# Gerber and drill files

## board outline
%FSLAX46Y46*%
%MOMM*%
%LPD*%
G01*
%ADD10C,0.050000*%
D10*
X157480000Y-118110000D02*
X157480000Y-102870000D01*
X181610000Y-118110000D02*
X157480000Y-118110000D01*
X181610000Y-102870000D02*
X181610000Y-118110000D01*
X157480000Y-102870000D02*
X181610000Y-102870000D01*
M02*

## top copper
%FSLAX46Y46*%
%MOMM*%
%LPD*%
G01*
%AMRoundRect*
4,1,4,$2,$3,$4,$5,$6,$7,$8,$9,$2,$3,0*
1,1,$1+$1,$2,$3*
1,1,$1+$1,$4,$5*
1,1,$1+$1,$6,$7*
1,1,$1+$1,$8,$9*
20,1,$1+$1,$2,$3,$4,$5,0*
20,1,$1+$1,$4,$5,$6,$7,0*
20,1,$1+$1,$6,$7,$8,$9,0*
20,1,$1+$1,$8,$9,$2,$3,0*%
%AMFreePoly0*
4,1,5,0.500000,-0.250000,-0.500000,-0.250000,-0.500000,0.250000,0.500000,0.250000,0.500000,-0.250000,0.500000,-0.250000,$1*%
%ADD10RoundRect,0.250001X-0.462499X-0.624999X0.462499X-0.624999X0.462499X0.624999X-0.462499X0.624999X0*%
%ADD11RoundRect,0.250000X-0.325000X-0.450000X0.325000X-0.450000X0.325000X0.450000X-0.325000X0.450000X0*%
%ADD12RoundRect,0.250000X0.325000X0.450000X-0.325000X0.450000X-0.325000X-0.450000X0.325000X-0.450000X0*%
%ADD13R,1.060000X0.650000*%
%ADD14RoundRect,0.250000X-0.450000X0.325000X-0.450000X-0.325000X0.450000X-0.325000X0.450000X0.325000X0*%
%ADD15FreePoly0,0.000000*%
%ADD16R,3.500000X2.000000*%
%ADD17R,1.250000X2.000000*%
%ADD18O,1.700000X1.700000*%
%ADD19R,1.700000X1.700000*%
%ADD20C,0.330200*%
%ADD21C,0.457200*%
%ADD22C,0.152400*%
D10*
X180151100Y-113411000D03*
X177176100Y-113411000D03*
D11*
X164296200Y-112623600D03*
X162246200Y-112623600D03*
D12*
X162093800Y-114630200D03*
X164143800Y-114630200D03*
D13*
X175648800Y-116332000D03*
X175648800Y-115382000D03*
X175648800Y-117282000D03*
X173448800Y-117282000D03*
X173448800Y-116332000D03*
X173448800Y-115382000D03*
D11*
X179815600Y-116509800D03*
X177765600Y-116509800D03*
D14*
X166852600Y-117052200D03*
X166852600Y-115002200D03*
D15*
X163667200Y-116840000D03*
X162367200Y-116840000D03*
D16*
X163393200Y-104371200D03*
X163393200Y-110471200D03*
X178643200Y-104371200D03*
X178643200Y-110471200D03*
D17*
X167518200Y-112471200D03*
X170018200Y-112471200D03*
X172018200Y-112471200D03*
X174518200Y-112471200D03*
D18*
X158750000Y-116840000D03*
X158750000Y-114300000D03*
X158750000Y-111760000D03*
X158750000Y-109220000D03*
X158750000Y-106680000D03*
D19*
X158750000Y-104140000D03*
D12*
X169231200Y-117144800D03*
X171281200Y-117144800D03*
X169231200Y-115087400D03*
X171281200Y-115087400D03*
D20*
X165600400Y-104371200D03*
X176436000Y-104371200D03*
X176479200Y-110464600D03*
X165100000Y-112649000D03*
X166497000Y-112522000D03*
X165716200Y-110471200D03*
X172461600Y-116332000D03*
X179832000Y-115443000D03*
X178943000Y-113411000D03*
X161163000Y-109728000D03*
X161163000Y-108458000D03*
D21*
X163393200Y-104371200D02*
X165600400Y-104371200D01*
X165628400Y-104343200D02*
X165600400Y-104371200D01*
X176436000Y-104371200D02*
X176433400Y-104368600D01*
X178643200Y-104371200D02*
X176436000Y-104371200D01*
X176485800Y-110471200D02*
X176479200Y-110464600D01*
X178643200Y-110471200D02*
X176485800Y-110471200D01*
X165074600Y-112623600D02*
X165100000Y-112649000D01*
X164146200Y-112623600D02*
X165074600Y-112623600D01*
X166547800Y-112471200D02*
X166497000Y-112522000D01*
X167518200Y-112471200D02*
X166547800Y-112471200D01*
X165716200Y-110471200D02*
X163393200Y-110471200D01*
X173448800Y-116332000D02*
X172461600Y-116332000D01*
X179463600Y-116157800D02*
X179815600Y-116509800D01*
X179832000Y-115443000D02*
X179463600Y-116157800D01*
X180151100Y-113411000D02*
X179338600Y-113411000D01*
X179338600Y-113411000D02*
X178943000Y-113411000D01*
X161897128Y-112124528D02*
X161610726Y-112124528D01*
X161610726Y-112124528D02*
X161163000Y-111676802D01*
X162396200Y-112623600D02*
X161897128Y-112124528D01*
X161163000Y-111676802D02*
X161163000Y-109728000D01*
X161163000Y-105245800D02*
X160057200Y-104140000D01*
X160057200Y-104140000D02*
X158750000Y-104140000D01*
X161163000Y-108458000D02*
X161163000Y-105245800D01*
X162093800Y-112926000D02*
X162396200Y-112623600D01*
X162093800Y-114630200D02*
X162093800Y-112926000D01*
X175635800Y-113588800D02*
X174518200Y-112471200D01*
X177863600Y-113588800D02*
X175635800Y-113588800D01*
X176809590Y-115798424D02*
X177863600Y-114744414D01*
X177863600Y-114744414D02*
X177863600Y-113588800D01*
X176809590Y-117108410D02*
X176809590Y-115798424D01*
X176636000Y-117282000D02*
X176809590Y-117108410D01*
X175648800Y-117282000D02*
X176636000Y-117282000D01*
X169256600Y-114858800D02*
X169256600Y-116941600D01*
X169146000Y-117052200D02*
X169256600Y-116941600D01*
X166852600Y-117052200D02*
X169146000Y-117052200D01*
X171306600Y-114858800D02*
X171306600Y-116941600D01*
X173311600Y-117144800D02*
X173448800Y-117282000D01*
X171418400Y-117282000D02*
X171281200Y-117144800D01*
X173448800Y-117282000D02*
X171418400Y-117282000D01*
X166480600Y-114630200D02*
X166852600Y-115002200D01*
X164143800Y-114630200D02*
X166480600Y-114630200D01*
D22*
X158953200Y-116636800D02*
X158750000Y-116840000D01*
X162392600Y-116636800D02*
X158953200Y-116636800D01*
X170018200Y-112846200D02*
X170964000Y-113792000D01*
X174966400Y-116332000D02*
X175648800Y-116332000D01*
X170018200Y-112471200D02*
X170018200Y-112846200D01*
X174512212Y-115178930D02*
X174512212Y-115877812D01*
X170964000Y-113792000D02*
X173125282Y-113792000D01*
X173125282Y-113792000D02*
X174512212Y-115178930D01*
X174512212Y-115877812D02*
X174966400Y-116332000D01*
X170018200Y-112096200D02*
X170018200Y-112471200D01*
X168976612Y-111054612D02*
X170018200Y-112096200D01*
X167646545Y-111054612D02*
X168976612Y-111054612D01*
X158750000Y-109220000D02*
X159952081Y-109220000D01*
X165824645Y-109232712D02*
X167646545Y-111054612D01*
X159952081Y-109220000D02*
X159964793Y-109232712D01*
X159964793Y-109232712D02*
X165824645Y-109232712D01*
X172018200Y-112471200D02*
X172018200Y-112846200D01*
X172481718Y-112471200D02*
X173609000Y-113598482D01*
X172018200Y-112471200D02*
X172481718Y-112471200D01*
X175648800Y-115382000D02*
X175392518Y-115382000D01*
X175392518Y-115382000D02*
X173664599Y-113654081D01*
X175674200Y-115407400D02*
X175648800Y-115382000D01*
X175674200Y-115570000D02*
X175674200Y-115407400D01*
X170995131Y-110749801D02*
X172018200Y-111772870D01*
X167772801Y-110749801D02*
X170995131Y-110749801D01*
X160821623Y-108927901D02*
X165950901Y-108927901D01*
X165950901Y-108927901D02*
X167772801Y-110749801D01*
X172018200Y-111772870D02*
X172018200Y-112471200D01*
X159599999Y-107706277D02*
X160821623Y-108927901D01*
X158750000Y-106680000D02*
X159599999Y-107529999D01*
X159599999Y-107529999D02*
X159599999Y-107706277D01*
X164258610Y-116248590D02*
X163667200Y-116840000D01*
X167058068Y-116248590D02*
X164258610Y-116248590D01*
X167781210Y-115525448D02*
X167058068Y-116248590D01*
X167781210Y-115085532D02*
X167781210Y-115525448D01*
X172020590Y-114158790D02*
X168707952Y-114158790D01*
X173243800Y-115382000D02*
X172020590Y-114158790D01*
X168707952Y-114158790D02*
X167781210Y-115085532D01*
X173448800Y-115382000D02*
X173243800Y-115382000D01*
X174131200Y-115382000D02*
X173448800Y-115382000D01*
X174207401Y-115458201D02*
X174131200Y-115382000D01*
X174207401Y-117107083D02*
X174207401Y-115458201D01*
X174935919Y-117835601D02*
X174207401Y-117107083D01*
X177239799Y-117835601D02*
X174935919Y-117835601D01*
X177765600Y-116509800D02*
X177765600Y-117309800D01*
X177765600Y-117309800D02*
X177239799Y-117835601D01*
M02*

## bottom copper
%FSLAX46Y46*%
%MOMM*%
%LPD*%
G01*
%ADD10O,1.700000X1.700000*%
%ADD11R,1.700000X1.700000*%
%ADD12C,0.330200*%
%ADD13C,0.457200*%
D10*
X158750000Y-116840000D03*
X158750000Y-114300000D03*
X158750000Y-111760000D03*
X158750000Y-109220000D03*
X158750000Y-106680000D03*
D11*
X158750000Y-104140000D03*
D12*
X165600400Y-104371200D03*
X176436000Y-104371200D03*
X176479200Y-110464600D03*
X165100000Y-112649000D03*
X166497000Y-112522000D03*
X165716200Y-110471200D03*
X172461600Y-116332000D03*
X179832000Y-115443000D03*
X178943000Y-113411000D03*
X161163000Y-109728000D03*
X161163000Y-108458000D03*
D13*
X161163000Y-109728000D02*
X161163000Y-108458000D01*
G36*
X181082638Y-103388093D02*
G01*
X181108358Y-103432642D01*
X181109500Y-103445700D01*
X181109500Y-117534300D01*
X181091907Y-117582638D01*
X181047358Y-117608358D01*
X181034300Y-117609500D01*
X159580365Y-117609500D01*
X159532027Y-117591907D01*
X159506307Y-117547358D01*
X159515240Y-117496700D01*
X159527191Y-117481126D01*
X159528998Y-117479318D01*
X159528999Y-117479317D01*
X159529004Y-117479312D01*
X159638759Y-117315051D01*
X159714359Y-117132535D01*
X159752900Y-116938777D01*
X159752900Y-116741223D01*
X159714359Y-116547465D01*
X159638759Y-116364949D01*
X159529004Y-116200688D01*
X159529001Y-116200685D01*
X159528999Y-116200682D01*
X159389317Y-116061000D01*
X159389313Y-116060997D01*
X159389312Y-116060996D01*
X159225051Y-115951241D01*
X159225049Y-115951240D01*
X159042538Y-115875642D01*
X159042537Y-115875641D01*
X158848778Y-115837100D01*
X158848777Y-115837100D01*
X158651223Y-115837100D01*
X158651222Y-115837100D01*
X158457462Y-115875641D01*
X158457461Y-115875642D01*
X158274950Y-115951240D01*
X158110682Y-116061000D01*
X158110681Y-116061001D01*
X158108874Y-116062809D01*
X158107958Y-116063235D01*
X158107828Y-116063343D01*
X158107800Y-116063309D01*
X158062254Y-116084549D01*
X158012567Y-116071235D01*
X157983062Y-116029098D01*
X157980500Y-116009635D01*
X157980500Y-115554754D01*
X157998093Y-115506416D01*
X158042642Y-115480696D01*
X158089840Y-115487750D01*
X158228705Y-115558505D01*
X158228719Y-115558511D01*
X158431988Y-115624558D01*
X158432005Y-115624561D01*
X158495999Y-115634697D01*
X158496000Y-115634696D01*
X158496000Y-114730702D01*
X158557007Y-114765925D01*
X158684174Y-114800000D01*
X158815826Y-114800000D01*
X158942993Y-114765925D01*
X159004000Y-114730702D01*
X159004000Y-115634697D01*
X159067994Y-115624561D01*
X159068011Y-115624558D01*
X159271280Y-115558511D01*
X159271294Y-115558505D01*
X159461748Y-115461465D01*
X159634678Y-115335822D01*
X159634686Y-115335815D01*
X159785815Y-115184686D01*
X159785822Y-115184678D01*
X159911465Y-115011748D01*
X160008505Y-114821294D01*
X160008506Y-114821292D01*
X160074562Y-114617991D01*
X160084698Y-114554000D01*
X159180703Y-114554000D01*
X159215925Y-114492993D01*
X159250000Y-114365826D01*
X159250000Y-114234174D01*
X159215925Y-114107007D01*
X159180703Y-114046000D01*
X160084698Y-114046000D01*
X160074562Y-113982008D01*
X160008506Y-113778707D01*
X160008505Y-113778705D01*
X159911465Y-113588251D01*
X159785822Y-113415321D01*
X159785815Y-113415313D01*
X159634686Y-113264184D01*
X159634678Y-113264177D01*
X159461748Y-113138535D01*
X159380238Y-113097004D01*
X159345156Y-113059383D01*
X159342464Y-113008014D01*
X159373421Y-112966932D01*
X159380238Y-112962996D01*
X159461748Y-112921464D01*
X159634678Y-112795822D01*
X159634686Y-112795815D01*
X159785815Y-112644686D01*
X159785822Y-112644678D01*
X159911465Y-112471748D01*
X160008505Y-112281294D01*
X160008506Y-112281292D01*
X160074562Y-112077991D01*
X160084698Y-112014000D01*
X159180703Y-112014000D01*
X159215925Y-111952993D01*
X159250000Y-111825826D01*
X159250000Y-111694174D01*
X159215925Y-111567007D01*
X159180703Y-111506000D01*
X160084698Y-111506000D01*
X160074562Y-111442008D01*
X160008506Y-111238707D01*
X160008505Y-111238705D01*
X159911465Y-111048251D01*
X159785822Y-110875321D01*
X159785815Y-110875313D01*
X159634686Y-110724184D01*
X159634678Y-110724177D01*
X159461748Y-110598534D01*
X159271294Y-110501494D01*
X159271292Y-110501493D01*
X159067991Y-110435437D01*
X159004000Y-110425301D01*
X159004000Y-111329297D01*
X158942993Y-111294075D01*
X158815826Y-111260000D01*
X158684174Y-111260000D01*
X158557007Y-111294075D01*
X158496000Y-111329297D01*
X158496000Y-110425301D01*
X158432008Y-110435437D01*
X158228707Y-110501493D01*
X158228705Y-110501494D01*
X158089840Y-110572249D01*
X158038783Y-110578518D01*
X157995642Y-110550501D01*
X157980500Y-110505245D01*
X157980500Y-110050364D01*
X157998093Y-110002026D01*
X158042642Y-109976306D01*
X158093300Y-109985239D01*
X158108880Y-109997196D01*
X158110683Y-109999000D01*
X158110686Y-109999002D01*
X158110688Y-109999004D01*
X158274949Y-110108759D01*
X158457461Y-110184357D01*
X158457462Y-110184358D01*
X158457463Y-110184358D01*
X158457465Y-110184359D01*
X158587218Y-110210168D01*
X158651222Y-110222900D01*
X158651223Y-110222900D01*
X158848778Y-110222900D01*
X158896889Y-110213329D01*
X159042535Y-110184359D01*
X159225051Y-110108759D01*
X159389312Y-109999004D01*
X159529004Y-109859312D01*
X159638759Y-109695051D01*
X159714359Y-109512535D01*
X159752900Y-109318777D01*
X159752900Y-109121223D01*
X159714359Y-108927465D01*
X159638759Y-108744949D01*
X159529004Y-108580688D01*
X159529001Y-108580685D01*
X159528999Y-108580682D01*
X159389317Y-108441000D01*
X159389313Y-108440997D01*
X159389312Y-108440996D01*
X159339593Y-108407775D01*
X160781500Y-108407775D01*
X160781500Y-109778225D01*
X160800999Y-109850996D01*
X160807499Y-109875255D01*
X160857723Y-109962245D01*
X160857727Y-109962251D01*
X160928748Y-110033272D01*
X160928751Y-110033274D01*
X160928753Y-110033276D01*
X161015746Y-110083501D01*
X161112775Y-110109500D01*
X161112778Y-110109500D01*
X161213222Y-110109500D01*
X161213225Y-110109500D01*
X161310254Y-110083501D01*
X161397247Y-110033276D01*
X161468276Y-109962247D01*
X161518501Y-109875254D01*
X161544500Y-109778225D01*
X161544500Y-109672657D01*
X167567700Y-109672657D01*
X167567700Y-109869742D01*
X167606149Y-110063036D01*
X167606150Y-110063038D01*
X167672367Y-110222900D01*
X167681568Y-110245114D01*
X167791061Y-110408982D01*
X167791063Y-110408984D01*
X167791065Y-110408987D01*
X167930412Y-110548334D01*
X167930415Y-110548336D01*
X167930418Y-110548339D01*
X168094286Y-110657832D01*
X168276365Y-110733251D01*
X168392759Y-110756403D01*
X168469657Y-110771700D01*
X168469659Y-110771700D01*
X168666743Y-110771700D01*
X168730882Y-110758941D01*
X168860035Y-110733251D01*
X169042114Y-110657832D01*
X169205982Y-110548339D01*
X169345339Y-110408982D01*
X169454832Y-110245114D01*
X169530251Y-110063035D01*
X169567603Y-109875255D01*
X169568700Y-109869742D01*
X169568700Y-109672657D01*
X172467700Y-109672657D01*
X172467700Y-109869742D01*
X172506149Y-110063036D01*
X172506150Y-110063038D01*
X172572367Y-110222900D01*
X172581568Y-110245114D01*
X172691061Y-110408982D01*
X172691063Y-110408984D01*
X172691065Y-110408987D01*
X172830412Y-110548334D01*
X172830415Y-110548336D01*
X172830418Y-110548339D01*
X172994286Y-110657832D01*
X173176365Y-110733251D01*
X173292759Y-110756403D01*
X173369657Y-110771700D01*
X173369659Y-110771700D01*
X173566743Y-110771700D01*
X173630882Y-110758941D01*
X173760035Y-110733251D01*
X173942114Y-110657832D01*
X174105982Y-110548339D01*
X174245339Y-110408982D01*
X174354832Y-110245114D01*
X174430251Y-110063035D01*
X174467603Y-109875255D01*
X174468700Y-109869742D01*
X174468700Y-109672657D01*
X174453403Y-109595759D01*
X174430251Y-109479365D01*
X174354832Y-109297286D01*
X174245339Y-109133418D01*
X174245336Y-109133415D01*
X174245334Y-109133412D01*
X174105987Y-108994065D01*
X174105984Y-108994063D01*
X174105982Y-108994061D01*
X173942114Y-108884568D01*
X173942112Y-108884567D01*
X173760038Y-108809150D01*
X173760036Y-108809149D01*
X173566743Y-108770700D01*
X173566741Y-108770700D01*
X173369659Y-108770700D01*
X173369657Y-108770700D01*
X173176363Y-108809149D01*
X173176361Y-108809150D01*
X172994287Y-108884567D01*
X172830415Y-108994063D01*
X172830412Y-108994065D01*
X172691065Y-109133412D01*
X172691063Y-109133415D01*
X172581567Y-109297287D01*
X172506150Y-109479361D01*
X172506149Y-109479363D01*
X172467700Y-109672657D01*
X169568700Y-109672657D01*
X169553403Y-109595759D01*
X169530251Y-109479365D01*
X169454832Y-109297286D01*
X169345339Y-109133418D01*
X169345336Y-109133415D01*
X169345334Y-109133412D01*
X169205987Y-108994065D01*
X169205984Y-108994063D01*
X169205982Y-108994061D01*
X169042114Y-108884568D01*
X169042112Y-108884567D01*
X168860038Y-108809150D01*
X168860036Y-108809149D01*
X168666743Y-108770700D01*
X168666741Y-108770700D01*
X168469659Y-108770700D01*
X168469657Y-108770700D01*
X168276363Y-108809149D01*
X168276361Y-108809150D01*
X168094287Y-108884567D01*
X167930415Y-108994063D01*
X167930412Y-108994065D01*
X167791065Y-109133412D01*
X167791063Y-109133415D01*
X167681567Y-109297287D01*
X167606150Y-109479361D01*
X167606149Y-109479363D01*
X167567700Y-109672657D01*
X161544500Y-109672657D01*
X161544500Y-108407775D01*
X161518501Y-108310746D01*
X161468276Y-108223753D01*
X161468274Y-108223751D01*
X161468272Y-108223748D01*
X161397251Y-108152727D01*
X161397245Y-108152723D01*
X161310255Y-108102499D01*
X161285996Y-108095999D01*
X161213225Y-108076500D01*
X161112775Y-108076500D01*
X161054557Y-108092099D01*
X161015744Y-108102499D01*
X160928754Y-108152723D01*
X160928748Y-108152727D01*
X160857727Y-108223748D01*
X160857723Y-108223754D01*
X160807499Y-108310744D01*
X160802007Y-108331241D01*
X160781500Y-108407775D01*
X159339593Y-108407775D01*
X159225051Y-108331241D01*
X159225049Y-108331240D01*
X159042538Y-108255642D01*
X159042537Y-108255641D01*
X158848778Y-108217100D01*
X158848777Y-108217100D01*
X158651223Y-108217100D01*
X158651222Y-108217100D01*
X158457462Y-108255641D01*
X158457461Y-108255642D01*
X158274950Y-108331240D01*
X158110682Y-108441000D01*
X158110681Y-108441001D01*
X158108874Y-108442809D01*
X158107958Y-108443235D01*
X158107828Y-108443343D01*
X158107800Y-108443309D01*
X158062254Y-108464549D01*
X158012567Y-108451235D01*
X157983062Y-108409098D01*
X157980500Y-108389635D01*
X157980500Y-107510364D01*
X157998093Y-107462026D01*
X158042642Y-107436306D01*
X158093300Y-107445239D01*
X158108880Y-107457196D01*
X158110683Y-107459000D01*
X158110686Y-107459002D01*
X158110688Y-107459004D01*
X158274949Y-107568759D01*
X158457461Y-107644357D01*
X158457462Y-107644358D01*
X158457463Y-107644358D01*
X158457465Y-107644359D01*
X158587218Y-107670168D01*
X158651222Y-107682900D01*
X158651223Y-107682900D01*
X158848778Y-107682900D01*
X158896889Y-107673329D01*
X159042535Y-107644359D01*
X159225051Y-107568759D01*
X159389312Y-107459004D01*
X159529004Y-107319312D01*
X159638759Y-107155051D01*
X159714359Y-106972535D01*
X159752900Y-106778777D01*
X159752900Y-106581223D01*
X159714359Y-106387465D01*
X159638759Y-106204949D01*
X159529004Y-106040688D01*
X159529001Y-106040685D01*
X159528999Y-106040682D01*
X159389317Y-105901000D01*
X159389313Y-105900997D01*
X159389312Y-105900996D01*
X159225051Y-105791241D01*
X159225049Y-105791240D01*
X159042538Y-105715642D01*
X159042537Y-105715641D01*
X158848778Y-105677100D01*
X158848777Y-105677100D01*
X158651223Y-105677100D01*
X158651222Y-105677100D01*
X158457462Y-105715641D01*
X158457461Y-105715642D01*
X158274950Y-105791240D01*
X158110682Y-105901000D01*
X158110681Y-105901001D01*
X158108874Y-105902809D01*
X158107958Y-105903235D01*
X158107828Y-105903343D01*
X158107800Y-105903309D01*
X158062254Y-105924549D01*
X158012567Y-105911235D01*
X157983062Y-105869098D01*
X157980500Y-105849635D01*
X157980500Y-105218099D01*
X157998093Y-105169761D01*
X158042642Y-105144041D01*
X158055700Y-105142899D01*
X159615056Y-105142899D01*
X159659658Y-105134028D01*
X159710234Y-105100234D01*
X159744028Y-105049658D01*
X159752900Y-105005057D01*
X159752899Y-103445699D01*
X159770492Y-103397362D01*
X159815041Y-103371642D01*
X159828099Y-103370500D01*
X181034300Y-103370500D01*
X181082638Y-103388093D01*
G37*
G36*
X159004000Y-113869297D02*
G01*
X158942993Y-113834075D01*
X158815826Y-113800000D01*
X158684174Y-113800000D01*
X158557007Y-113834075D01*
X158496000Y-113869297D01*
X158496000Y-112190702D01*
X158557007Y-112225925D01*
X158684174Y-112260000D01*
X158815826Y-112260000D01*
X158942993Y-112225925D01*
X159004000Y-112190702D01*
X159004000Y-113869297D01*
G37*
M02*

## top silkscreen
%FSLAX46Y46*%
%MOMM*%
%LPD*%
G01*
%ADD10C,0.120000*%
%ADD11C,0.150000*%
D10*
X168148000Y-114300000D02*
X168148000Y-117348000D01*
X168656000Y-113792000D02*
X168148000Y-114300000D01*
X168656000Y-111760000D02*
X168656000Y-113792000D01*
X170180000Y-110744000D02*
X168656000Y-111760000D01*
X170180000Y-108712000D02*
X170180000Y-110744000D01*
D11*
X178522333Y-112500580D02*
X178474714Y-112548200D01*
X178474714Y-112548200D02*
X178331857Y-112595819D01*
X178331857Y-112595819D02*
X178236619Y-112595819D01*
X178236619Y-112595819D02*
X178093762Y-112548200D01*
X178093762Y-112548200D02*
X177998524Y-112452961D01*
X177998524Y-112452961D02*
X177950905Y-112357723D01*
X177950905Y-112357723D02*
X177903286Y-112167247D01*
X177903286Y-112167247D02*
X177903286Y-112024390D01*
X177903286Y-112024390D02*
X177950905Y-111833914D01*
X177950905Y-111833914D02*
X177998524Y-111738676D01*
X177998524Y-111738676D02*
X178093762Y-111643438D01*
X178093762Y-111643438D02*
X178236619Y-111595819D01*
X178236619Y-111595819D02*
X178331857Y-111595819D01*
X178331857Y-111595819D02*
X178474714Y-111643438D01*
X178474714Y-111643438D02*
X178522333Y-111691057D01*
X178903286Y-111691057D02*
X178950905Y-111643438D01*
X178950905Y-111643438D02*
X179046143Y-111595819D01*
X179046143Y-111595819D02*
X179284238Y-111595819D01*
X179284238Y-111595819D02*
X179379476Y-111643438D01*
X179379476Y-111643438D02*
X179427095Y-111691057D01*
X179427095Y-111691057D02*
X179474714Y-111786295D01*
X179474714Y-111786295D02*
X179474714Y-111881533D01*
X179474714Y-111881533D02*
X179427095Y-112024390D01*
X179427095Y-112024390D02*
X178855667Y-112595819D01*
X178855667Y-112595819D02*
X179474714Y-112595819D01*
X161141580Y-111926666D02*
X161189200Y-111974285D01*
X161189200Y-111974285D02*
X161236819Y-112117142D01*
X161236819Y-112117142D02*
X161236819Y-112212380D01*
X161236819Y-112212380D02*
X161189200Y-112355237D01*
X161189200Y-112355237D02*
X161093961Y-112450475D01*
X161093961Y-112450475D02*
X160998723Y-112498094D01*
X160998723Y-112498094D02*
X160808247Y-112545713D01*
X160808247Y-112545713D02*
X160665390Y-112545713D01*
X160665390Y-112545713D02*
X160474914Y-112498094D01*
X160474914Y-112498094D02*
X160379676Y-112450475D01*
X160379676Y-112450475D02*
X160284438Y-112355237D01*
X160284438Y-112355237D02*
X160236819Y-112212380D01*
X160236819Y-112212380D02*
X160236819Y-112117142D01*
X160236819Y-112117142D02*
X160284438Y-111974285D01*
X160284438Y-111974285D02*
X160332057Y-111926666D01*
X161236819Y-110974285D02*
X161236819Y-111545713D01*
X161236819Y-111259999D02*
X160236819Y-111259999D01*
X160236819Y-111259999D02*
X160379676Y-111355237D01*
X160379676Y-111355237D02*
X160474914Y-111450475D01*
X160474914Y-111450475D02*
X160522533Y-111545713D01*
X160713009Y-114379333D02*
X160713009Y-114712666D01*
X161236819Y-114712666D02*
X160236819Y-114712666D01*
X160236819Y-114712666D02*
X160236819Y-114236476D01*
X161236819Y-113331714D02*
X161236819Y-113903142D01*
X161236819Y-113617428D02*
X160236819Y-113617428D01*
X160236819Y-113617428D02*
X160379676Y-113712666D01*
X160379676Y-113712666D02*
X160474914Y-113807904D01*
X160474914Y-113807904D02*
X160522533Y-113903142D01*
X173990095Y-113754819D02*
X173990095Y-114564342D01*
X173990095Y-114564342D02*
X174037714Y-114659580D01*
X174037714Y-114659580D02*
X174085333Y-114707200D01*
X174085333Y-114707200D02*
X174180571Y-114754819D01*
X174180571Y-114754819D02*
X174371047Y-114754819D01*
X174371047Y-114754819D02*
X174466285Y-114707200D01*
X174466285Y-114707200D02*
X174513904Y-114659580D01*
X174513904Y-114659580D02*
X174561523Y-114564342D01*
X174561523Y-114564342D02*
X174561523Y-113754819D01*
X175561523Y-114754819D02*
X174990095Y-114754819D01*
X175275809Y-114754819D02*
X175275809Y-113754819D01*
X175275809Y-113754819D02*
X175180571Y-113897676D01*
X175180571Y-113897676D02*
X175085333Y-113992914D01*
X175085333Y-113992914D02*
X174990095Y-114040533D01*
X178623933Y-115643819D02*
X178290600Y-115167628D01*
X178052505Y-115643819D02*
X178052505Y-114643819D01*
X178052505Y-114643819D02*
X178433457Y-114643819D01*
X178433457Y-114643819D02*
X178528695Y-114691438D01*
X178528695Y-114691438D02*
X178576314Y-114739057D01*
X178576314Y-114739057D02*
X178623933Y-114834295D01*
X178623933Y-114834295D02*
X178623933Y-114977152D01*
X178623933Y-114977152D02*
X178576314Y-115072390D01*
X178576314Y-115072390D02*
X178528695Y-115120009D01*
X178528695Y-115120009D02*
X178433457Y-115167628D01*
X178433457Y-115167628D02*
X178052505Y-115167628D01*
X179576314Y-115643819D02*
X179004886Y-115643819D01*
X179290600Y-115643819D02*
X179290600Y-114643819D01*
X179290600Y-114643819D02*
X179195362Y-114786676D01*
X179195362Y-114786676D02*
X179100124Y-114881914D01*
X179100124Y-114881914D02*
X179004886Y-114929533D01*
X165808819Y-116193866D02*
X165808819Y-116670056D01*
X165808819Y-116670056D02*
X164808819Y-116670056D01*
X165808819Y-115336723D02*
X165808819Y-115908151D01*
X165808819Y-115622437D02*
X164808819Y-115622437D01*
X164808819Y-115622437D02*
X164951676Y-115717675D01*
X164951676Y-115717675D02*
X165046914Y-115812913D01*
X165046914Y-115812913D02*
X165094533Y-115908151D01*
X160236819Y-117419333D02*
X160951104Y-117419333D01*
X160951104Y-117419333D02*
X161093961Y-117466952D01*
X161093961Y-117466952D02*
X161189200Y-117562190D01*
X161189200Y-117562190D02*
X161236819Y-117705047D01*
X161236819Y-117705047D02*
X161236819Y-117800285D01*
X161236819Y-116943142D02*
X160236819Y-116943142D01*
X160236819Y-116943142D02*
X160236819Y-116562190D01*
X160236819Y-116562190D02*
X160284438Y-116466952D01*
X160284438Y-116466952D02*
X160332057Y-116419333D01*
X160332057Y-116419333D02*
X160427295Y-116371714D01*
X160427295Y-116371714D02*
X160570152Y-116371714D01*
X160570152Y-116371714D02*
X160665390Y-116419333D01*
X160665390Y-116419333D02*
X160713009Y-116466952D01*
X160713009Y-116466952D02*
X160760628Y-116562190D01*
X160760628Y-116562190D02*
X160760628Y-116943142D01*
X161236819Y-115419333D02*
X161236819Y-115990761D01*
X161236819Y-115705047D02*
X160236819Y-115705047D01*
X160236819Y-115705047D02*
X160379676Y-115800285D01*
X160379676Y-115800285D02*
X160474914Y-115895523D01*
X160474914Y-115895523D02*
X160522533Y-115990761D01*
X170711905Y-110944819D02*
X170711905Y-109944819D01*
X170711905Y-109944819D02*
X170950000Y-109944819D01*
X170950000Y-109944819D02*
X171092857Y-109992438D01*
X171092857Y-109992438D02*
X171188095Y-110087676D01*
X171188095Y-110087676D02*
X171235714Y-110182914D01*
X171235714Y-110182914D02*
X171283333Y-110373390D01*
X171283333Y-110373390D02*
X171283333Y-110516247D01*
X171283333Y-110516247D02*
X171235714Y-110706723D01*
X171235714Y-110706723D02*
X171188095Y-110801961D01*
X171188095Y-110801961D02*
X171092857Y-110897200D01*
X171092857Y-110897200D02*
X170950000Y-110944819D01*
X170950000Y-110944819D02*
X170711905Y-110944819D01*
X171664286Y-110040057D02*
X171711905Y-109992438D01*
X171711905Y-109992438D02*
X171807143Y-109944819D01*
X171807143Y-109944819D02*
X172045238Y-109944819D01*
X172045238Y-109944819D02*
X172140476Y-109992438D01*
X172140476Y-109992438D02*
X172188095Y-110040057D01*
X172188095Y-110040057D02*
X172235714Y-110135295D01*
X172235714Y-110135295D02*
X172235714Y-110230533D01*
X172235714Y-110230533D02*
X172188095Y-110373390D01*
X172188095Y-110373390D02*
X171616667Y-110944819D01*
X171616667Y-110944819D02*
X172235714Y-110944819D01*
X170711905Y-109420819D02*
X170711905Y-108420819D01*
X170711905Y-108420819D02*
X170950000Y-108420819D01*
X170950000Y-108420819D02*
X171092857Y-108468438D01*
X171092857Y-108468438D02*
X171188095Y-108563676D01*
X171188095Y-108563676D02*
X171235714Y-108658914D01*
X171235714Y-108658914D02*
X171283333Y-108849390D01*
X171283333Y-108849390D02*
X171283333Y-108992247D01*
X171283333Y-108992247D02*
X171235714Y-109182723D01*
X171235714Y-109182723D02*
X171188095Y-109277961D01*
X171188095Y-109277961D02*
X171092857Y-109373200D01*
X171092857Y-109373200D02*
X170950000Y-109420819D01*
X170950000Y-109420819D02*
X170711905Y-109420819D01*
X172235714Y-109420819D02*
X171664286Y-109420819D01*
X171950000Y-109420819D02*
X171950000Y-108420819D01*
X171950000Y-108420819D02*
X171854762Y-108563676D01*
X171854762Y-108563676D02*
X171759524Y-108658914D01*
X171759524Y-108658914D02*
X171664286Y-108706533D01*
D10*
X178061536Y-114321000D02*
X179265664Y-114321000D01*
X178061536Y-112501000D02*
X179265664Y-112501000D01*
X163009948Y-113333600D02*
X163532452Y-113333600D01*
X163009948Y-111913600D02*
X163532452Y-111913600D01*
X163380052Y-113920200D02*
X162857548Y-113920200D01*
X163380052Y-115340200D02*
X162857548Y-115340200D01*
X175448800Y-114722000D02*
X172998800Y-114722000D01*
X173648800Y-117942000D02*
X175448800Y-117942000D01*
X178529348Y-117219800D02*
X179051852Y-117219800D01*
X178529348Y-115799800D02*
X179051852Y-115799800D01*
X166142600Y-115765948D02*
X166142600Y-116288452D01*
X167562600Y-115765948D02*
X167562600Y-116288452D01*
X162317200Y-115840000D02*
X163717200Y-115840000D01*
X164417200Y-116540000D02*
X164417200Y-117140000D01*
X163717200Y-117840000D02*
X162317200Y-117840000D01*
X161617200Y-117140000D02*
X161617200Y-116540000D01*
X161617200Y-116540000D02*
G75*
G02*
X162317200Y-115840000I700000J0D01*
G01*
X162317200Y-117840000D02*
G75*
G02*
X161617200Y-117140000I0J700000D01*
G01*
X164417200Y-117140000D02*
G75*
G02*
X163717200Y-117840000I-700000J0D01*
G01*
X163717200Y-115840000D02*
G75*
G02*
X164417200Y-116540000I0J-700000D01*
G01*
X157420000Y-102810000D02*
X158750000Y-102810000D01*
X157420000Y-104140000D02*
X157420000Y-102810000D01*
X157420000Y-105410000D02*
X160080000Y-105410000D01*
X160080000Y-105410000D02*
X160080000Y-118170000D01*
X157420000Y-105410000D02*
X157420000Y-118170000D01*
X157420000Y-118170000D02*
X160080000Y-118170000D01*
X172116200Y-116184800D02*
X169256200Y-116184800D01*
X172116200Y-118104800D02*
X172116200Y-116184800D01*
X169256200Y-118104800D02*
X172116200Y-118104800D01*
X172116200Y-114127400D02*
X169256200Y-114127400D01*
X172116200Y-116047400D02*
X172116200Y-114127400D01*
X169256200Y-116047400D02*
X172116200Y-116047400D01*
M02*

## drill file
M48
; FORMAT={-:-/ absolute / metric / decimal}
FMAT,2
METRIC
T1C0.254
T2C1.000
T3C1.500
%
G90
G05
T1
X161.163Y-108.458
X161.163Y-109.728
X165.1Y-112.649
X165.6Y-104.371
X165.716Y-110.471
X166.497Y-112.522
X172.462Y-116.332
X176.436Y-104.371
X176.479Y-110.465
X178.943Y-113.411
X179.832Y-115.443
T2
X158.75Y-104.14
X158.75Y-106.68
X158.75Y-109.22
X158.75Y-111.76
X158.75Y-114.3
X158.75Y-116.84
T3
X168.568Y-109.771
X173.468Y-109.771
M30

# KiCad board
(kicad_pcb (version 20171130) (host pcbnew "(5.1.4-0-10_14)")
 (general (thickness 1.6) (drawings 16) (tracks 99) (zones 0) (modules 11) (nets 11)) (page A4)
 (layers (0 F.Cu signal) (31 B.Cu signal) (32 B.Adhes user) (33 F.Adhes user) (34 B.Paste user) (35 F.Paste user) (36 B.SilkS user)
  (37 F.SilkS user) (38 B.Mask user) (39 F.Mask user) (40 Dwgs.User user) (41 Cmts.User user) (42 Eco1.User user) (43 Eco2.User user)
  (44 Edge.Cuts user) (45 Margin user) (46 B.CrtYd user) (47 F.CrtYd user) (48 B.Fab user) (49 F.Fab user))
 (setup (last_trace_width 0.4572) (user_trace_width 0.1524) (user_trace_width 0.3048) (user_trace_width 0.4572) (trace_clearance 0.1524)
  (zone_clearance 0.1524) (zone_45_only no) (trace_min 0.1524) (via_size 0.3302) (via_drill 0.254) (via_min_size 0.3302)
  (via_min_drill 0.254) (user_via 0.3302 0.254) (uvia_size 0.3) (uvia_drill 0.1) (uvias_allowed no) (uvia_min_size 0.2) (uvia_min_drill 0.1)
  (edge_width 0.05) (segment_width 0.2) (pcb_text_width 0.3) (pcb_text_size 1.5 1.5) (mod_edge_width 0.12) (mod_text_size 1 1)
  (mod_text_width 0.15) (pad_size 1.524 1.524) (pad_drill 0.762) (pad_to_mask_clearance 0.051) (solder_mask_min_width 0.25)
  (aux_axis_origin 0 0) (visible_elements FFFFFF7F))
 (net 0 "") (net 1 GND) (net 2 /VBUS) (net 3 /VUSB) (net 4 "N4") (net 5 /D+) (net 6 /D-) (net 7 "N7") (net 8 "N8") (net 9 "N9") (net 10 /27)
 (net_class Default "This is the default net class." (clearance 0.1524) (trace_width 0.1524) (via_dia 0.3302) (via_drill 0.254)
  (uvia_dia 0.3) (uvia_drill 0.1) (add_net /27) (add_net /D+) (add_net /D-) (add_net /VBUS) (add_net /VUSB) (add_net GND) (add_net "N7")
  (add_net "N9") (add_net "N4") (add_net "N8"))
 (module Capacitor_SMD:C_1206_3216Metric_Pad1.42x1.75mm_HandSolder (layer F.Cu) (at 178.6636 113.411)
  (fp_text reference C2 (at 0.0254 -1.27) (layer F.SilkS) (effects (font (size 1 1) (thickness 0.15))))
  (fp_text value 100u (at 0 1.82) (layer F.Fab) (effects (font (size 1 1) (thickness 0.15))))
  (fp_line (start -0.602064 0.91) (end 0.602064 0.91) (layer F.SilkS) (width 0.12))
  (fp_line (start -0.602064 -0.91) (end 0.602064 -0.91) (layer F.SilkS) (width 0.12))
  (pad 2 smd roundrect (at 1.4875 0) (size 1.425 1.75) (layers F.Cu F.Paste F.Mask) (roundrect_rratio 0.175439) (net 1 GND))
  (pad 1 smd roundrect (at -1.4875 0) (size 1.425 1.75) (layers F.Cu F.Paste F.Mask) (roundrect_rratio 0.175439) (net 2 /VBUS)))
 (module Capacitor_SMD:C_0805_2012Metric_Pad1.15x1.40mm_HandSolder (layer F.Cu) (at 163.2712 112.6236)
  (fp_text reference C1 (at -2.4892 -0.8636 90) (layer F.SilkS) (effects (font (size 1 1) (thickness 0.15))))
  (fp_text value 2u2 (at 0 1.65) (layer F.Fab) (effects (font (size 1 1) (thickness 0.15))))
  (fp_line (start -0.261252 0.71) (end 0.261252 0.71) (layer F.SilkS) (width 0.12))
  (fp_line (start -0.261252 -0.71) (end 0.261252 -0.71) (layer F.SilkS) (width 0.12))
  (pad 2 smd roundrect (at 1.025 0) (size 1.15 1.4) (layers F.Cu F.Paste F.Mask) (roundrect_rratio 0.217391) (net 1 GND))
  (pad 1 smd roundrect (at -1.025 0) (size 1.15 1.4) (layers F.Cu F.Paste F.Mask) (roundrect_rratio 0.217391) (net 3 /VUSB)))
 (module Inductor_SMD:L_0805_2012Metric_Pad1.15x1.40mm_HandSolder (layer F.Cu) (at 163.1188 114.6302 180)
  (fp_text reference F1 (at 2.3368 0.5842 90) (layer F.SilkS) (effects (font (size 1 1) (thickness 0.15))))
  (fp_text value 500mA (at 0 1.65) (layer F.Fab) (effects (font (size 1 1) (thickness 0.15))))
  (fp_line (start -0.261252 0.71) (end 0.261252 0.71) (layer F.SilkS) (width 0.12))
  (fp_line (start -0.261252 -0.71) (end 0.261252 -0.71) (layer F.SilkS) (width 0.12))
  (pad 2 smd roundrect (at 1.025 0 180) (size 1.15 1.4) (layers F.Cu F.Paste F.Mask) (roundrect_rratio 0.217391) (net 3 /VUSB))
  (pad 1 smd roundrect (at -1.025 0 180) (size 1.15 1.4) (layers F.Cu F.Paste F.Mask) (roundrect_rratio 0.217391) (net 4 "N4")))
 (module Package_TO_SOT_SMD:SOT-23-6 (layer F.Cu) (at 174.5488 116.332)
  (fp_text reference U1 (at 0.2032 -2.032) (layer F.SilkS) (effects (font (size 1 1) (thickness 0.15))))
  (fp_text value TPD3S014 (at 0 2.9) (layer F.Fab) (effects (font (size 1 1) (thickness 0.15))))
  (fp_line (start 0.9 -1.61) (end -1.55 -1.61) (layer F.SilkS) (width 0.12))
  (fp_line (start -0.9 1.61) (end 0.9 1.61) (layer F.SilkS) (width 0.12))
  (pad 5 smd rect (at 1.1 0) (size 1.06 0.65) (layers F.Cu F.Paste F.Mask) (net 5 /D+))
  (pad 6 smd rect (at 1.1 -0.95) (size 1.06 0.65) (layers F.Cu F.Paste F.Mask) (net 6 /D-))
  (pad 4 smd rect (at 1.1 0.95) (size 1.06 0.65) (layers F.Cu F.Paste F.Mask) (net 2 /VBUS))
  (pad 3 smd rect (at -1.1 0.95) (size 1.06 0.65) (layers F.Cu F.Paste F.Mask) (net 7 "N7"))
  (pad 2 smd rect (at -1.1 0) (size 1.06 0.65) (layers F.Cu F.Paste F.Mask) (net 1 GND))
  (pad 1 smd rect (at -1.1 -0.95) (size 1.06 0.65) (layers F.Cu F.Paste F.Mask) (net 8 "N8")))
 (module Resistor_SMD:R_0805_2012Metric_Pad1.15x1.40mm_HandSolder (layer F.Cu) (at 178.7906 116.5098)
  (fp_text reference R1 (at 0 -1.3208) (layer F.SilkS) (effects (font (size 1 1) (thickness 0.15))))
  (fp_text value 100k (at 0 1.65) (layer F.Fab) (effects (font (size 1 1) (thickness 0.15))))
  (fp_line (start -0.261252 0.71) (end 0.261252 0.71) (layer F.SilkS) (width 0.12))
  (fp_line (start -0.261252 -0.71) (end 0.261252 -0.71) (layer F.SilkS) (width 0.12))
  (pad 2 smd roundrect (at 1.025 0) (size 1.15 1.4) (layers F.Cu F.Paste F.Mask) (roundrect_rratio 0.217391) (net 1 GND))
  (pad 1 smd roundrect (at -1.025 0) (size 1.15 1.4) (layers F.Cu F.Paste F.Mask) (roundrect_rratio 0.217391) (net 8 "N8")))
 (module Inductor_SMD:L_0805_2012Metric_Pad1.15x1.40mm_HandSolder (layer F.Cu) (at 166.8526 116.0272 270)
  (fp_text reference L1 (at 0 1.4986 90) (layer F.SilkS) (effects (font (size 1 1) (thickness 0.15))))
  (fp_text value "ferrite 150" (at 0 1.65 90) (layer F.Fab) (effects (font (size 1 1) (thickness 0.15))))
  (fp_line (start -0.261252 0.71) (end 0.261252 0.71) (layer F.SilkS) (width 0.12))
  (fp_line (start -0.261252 -0.71) (end 0.261252 -0.71) (layer F.SilkS) (width 0.12))
  (pad 2 smd roundrect (at 1.025 0 270) (size 1.15 1.4) (layers F.Cu F.Paste F.Mask) (roundrect_rratio 0.217391) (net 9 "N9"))
  (pad 1 smd roundrect (at -1.025 0 270) (size 1.15 1.4) (layers F.Cu F.Paste F.Mask) (roundrect_rratio 0.217391) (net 4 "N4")))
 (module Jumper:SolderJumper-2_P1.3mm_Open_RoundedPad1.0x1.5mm (layer F.Cu) (at 163.0172 116.84)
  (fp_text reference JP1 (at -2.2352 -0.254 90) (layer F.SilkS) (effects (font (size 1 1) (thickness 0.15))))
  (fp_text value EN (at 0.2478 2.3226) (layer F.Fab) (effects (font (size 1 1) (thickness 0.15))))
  (fp_line (start -0.7 -1) (end 0.7 -1) (layer F.SilkS) (width 0.12))
  (fp_line (start 1.4 -0.3) (end 1.4 0.3) (layer F.SilkS) (width 0.12))
  (fp_line (start 0.7 1) (end -0.7 1) (layer F.SilkS) (width 0.12))
  (fp_line (start -1.4 0.3) (end -1.4 -0.3) (layer F.SilkS) (width 0.12))
  (fp_arc (start -0.7 -0.3) (end -0.7 -1) (angle -90) (layer F.SilkS) (width 0.12))
  (fp_arc (start -0.7 0.3) (end -1.4 0.3) (angle -90) (layer F.SilkS) (width 0.12))
  (fp_arc (start 0.7 0.3) (end 0.7 1) (angle -90) (layer F.SilkS) (width 0.12))
  (fp_arc (start 0.7 -0.3) (end 1.4 -0.3) (angle -90) (layer F.SilkS) (width 0.12))
  (pad 2 smd custom (at 0.65 0) (size 1 0.5) (layers F.Cu F.Mask) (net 8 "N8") (zone_connect 2) (options (clearance outline) (anchor rect))
   (primitives))
  (pad 1 smd custom (at -0.65 0) (size 1 0.5) (layers F.Cu F.Mask) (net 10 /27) (zone_connect 2) (options (clearance outline) (anchor rect))
   (primitives)))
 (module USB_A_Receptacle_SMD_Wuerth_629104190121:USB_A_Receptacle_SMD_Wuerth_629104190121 (layer F.Cu) (at 171.0182 112.4712 180)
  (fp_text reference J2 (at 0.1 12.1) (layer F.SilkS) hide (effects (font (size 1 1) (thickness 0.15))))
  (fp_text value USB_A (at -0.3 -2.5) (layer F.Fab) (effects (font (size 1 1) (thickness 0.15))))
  (pad "" np_thru_hole circle (at 2.45 2.7 180) (size 1.5 1.5) (drill 1.5) (layers *.Cu *.Mask))
  (pad "" np_thru_hole circle (at -2.45 2.7 180) (size 1.5 1.5) (drill 1.5) (layers *.Cu *.Mask))
  (pad 5 smd rect (at 7.625 8.1 180) (size 3.5 2) (layers F.Cu F.Paste F.Mask) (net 1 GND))
  (pad 5 smd rect (at 7.625 2 180) (size 3.5 2) (layers F.Cu F.Paste F.Mask) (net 1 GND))
  (pad 5 smd rect (at -7.625 8.1 180) (size 3.5 2) (layers F.Cu F.Paste F.Mask) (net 1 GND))
  (pad 5 smd rect (at -7.625 2 180) (size 3.5 2) (layers F.Cu F.Paste F.Mask) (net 1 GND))
  (pad 4 smd rect (at 3.5 0 180) (size 1.25 2) (layers F.Cu F.Paste F.Mask) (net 1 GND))
  (pad 3 smd rect (at 1 0 180) (size 1.25 2) (layers F.Cu F.Paste F.Mask) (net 5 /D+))
  (pad 2 smd rect (at -1 0 180) (size 1.25 2) (layers F.Cu F.Paste F.Mask) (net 6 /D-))
  (pad 1 smd rect (at -3.5 0 180) (size 1.25 2) (layers F.Cu F.Paste F.Mask) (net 2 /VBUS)))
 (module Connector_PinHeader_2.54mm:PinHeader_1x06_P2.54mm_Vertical (layer F.Cu) (at 158.75 104.14)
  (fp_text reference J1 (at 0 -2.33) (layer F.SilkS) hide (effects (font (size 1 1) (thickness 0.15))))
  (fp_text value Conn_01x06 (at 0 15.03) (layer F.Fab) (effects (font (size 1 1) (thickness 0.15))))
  (fp_line (start -1.33 -1.33) (end 0 -1.33) (layer F.SilkS) (width 0.12))
  (fp_line (start -1.33 0) (end -1.33 -1.33) (layer F.SilkS) (width 0.12))
  (fp_line (start -1.33 1.27) (end 1.33 1.27) (layer F.SilkS) (width 0.12))
  (fp_line (start 1.33 1.27) (end 1.33 14.03) (layer F.SilkS) (width 0.12))
  (fp_line (start -1.33 1.27) (end -1.33 14.03) (layer F.SilkS) (width 0.12))
  (fp_line (start -1.33 14.03) (end 1.33 14.03) (layer F.SilkS) (width 0.12))
  (pad 6 thru_hole oval (at 0 12.7) (size 1.7 1.7) (drill 1) (layers *.Cu *.Mask) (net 10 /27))
  (pad 5 thru_hole oval (at 0 10.16) (size 1.7 1.7) (drill 1) (layers *.Cu *.Mask) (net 1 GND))
  (pad 4 thru_hole oval (at 0 7.62) (size 1.7 1.7) (drill 1) (layers *.Cu *.Mask) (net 1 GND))
  (pad 3 thru_hole oval (at 0 5.08) (size 1.7 1.7) (drill 1) (layers *.Cu *.Mask) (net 5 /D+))
  (pad 2 thru_hole oval (at 0 2.54) (size 1.7 1.7) (drill 1) (layers *.Cu *.Mask) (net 6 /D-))
  (pad 1 thru_hole rect (at 0 0) (size 1.7 1.7) (drill 1) (layers *.Cu *.Mask) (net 3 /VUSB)))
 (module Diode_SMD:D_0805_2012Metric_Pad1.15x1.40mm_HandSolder (layer F.Cu) (at 170.2562 117.1448 180)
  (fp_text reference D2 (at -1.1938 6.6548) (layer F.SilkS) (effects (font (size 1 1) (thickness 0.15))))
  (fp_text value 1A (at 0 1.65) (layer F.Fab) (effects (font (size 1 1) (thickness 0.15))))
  (fp_line (start -1.86 0.96) (end 1 0.96) (layer F.SilkS) (width 0.12))
  (fp_line (start -1.86 -0.96) (end -1.86 0.96) (layer F.SilkS) (width 0.12))
  (fp_line (start 1 -0.96) (end -1.86 -0.96) (layer F.SilkS) (width 0.12))
  (pad 2 smd roundrect (at 1.025 0 180) (size 1.15 1.4) (layers F.Cu F.Paste F.Mask) (roundrect_rratio 0.217391) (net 9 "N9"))
  (pad 1 smd roundrect (at -1.025 0 180) (size 1.15 1.4) (layers F.Cu F.Paste F.Mask) (roundrect_rratio 0.217391) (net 7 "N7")))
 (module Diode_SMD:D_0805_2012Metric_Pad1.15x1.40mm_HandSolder (layer F.Cu) (at 170.2562 115.0874 180)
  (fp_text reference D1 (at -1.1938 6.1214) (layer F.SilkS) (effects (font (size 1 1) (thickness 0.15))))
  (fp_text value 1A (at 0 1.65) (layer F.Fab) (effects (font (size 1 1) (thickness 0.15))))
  (fp_line (start -1.86 0.96) (end 1 0.96) (layer F.SilkS) (width 0.12))
  (fp_line (start -1.86 -0.96) (end -1.86 0.96) (layer F.SilkS) (width 0.12))
  (fp_line (start 1 -0.96) (end -1.86 -0.96) (layer F.SilkS) (width 0.12))
  (pad 2 smd roundrect (at 1.025 0 180) (size 1.15 1.4) (layers F.Cu F.Paste F.Mask) (roundrect_rratio 0.217391) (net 9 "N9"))
  (pad 1 smd roundrect (at -1.025 0 180) (size 1.15 1.4) (layers F.Cu F.Paste F.Mask) (roundrect_rratio 0.217391) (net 7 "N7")))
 (gr_line (start 168.148 114.3) (end 168.148 117.348) (layer F.SilkS) (width 0.12))
 (gr_line (start 168.656 113.792) (end 168.148 114.3) (layer F.SilkS) (width 0.12))
 (gr_line (start 168.656 111.76) (end 168.656 113.792) (layer F.SilkS) (width 0.12))
 (gr_line (start 170.18 110.744) (end 168.656 111.76) (layer F.SilkS) (width 0.12))
 (gr_line (start 170.18 108.712) (end 170.18 110.744) (layer F.SilkS) (width 0.12))
 (gr_line (start 157.48 118.11) (end 157.48 102.87) (layer Edge.Cuts) (width 0.05))
 (gr_line (start 181.61 118.11) (end 157.48 118.11) (layer Edge.Cuts) (width 0.05))
 (gr_line (start 181.61 102.87) (end 181.61 118.11) (layer Edge.Cuts) (width 0.05))
 (gr_line (start 157.48 102.87) (end 181.61 102.87) (layer Edge.Cuts) (width 0.05))
 (segment (start 163.3932 104.3712) (end 165.6004 104.3712) (width 0.4572) (layer F.Cu) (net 1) (status 10))
 (via (at 165.6004 104.3712) (size 0.3302) (drill 0.254) (layers F.Cu B.Cu) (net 1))
 (segment (start 165.6284 104.3432) (end 165.6004 104.3712) (width 0.4572) (layer F.Cu) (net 1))
 (segment (start 176.436 104.3712) (end 176.4334 104.3686) (width 0.4572) (layer F.Cu) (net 1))
 (segment (start 178.6432 104.3712) (end 176.436 104.3712) (width 0.4572) (layer F.Cu) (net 1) (status 10))
 (via (at 176.436 104.3712) (size 0.3302) (drill 0.254) (layers F.Cu B.Cu) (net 1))
 (via (at 176.4792 110.4646) (size 0.3302) (drill 0.254) (layers F.Cu B.Cu) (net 1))
 (segment (start 176.4858 110.4712) (end 176.4792 110.4646) (width 0.4572) (layer F.Cu) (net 1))
 (segment (start 178.6432 110.4712) (end 176.4858 110.4712) (width 0.4572) (layer F.Cu) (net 1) (status 10))
 (segment (start 165.0746 112.6236) (end 165.1 112.649) (width 0.4572) (layer F.Cu) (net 1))
 (via (at 165.1 112.649) (size 0.3302) (drill 0.254) (layers F.Cu B.Cu) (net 1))
 (segment (start 164.1462 112.6236) (end 165.0746 112.6236) (width 0.4572) (layer F.Cu) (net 1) (status 10))
 (via (at 166.497 112.522) (size 0.3302) (drill 0.254) (layers F.Cu B.Cu) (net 1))
 (segment (start 166.5478 112.4712) (end 166.497 112.522) (width 0.4572) (layer F.Cu) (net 1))
 (segment (start 167.5182 112.4712) (end 166.5478 112.4712) (width 0.4572) (layer F.Cu) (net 1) (status 10))
 (via (at 165.7162 110.4712) (size 0.3302) (drill 0.254) (layers F.Cu B.Cu) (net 1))
 (segment (start 165.7162 110.4712) (end 163.3932 110.4712) (width 0.4572) (layer F.Cu) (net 1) (status 20))
 (segment (start 173.4488 116.332) (end 172.4616 116.332) (width 0.4572) (layer F.Cu) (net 1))
 (via (at 172.4616 116.332) (size 0.3302) (drill 0.254) (layers F.Cu B.Cu) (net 1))
 (segment (start 179.4636 116.1578) (end 179.8156 116.5098) (width 0.4572) (layer F.Cu) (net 1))
 (segment (start 179.832 115.443) (end 179.4636 116.1578) (width 0.4572) (layer F.Cu) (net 1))
 (via (at 179.832 115.443) (size 0.3302) (drill 0.254) (layers F.Cu B.Cu) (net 1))
 (segment (start 180.1511 113.411) (end 179.3386 113.411) (width 0.4572) (layer F.Cu) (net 1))
 (via (at 178.943 113.411) (size 0.3302) (drill 0.254) (layers F.Cu B.Cu) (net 1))
 (segment (start 179.3386 113.411) (end 178.943 113.411) (width 0.4572) (layer F.Cu) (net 1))
 (segment (start 161.897128 112.124528) (end 161.610726 112.124528) (width 0.4572) (layer F.Cu) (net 3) (status 10))
 (segment (start 161.610726 112.124528) (end 161.163 111.676802) (width 0.4572) (layer F.Cu) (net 3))
 (segment (start 162.3962 112.6236) (end 161.897128 112.124528) (width 0.4572) (layer F.Cu) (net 3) (status 30))
 (via (at 161.163 109.728) (size 0.3302) (drill 0.254) (layers F.Cu B.Cu) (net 3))
 (segment (start 161.163 111.676802) (end 161.163 109.728) (width 0.4572) (layer F.Cu) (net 3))
 (segment (start 161.163 109.728) (end 161.163 108.458) (width 0.4572) (layer B.Cu) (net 3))
 (via (at 161.163 108.458) (size 0.3302) (drill 0.254) (layers F.Cu B.Cu) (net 3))
 (segment (start 161.163 105.2458) (end 160.0572 104.14) (width 0.4572) (layer F.Cu) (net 3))
 (segment (start 160.0572 104.14) (end 158.75 104.14) (width 0.4572) (layer F.Cu) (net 3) (status 20))
 (segment (start 161.163 108.458) (end 161.163 105.2458) (width 0.4572) (layer F.Cu) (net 3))
 (segment (start 162.0938 112.926) (end 162.3962 112.6236) (width 0.4572) (layer F.Cu) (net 3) (status 30))
 (segment (start 162.0938 114.6302) (end 162.0938 112.926) (width 0.4572) (layer F.Cu) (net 3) (status 30))
 (segment (start 175.6358 113.5888) (end 174.5182 112.4712) (width 0.4572) (layer F.Cu) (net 2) (status 20))
 (segment (start 177.8636 113.5888) (end 175.6358 113.5888) (width 0.4572) (layer F.Cu) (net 2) (status 10))
 (segment (start 176.80959 115.798424) (end 177.8636 114.744414) (width 0.4572) (layer F.Cu) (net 2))
 (segment (start 177.8636 114.744414) (end 177.8636 113.5888) (width 0.4572) (layer F.Cu) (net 2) (status 20))
 (segment (start 176.80959 117.10841) (end 176.80959 115.798424) (width 0.4572) (layer F.Cu) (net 2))
 (segment (start 176.636 117.282) (end 176.80959 117.10841) (width 0.4572) (layer F.Cu) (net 2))
 (segment (start 175.6488 117.282) (end 176.636 117.282) (width 0.4572) (layer F.Cu) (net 2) (status 10))
 (segment (start 169.2566 114.8588) (end 169.2566 116.9416) (width 0.4572) (layer F.Cu) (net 9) (status 30))
 (segment (start 169.146 117.0522) (end 169.2566 116.9416) (width 0.4572) (layer F.Cu) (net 9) (status 30))
 (segment (start 166.8526 117.0522) (end 169.146 117.0522) (width 0.4572) (layer F.Cu) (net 9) (status 30))
 (segment (start 171.3066 114.8588) (end 171.3066 116.9416) (width 0.4572) (layer F.Cu) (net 7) (status 30))
 (segment (start 173.3116 117.1448) (end 173.4488 117.282) (width 0.4572) (layer F.Cu) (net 7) (status 30))
 (segment (start 171.4184 117.282) (end 171.2812 117.1448) (width 0.4572) (layer F.Cu) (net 7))
 (segment (start 173.4488 117.282) (end 171.4184 117.282) (width 0.4572) (layer F.Cu) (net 7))
 (segment (start 166.4806 114.6302) (end 166.8526 115.0022) (width 0.4572) (layer F.Cu) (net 4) (status 30))
 (segment (start 164.1438 114.6302) (end 166.4806 114.6302) (width 0.4572) (layer F.Cu) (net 4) (status 30))
 (segment (start 158.9532 116.6368) (end 158.75 116.84) (width 0.1524) (layer F.Cu) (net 10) (status 30))
 (segment (start 162.3926 116.6368) (end 158.9532 116.6368) (width 0.1524) (layer F.Cu) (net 10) (status 30))
 (segment (start 170.0182 112.8462) (end 170.964 113.792) (width 0.1524) (layer F.Cu) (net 5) (status 10))
 (segment (start 174.9664 116.332) (end 175.6488 116.332) (width 0.1524) (layer F.Cu) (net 5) (status 20))
 (segment (start 170.0182 112.4712) (end 170.0182 112.8462) (width 0.1524) (layer F.Cu) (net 5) (status 30))
 (segment (start 174.512212 115.17893) (end 174.512212 115.877812) (width 0.1524) (layer F.Cu) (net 5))
 (segment (start 170.964 113.792) (end 173.125282 113.792) (width 0.1524) (layer F.Cu) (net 5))
 (segment (start 173.125282 113.792) (end 174.512212 115.17893) (width 0.1524) (layer F.Cu) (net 5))
 (segment (start 174.512212 115.877812) (end 174.9664 116.332) (width 0.1524) (layer F.Cu) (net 5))
 (segment (start 170.0182 112.0962) (end 170.0182 112.4712) (width 0.1524) (layer F.Cu) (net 5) (status 30))
 (segment (start 168.976612 111.054612) (end 170.0182 112.0962) (width 0.1524) (layer F.Cu) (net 5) (status 20))
 (segment (start 167.646545 111.054612) (end 168.976612 111.054612) (width 0.1524) (layer F.Cu) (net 5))
 (segment (start 158.75 109.22) (end 159.952081 109.22) (width 0.1524) (layer F.Cu) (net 5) (status 10))
 (segment (start 165.824645 109.232712) (end 167.646545 111.054612) (width 0.1524) (layer F.Cu) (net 5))
 (segment (start 159.952081 109.22) (end 159.964793 109.232712) (width 0.1524) (layer F.Cu) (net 5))
 (segment (start 159.964793 109.232712) (end 165.824645 109.232712) (width 0.1524) (layer F.Cu) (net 5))
 (segment (start 172.0182 112.4712) (end 172.0182 112.8462) (width 0.1524) (layer F.Cu) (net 6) (status 30))
 (segment (start 172.481718 112.4712) (end 173.609 113.598482) (width 0.1524) (layer F.Cu) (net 6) (status 10))
 (segment (start 172.0182 112.4712) (end 172.481718 112.4712) (width 0.1524) (layer F.Cu) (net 6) (status 30))
 (segment (start 175.6488 115.382) (end 175.392518 115.382) (width 0.1524) (layer F.Cu) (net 6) (status 30))
 (segment (start 175.392518 115.382) (end 173.664599 113.654081) (width 0.1524) (layer F.Cu) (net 6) (status 10))
 (segment (start 175.6742 115.4074) (end 175.6488 115.382) (width 0.1524) (layer F.Cu) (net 6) (status 30))
 (segment (start 175.6742 115.57) (end 175.6742 115.4074) (width 0.1524) (layer F.Cu) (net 6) (status 30))
 (segment (start 170.995131 110.749801) (end 172.0182 111.77287) (width 0.1524) (layer F.Cu) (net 6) (status 20))
 (segment (start 167.772801 110.749801) (end 170.995131 110.749801) (width 0.1524) (layer F.Cu) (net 6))
 (segment (start 160.821623 108.927901) (end 165.950901 108.927901) (width 0.1524) (layer F.Cu) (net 6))
 (segment (start 165.950901 108.927901) (end 167.772801 110.749801) (width 0.1524) (layer F.Cu) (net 6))
 (segment (start 172.0182 111.77287) (end 172.0182 112.4712) (width 0.1524) (layer F.Cu) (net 6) (status 30))
 (segment (start 159.599999 107.706277) (end 160.821623 108.927901) (width 0.1524) (layer F.Cu) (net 6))
 (segment (start 158.75 106.68) (end 159.599999 107.529999) (width 0.1524) (layer F.Cu) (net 6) (status 10))
 (segment (start 159.599999 107.529999) (end 159.599999 107.706277) (width 0.1524) (layer F.Cu) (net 6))
 (segment (start 164.25861 116.24859) (end 163.6672 116.84) (width 0.1524) (layer F.Cu) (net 8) (status 20))
 (segment (start 167.058068 116.24859) (end 164.25861 116.24859) (width 0.1524) (layer F.Cu) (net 8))
 (segment (start 167.78121 115.525448) (end 167.058068 116.24859) (width 0.1524) (layer F.Cu) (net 8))
 (segment (start 167.78121 115.085532) (end 167.78121 115.525448) (width 0.1524) (layer F.Cu) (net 8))
 (segment (start 172.02059 114.15879) (end 168.707952 114.15879) (width 0.1524) (layer F.Cu) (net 8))
 (segment (start 173.2438 115.382) (end 172.02059 114.15879) (width 0.1524) (layer F.Cu) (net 8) (status 10))
 (segment (start 168.707952 114.15879) (end 167.78121 115.085532) (width 0.1524) (layer F.Cu) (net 8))
 (segment (start 173.4488 115.382) (end 173.2438 115.382) (width 0.1524) (layer F.Cu) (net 8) (status 30))
 (segment (start 174.1312 115.382) (end 173.4488 115.382) (width 0.1524) (layer F.Cu) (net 8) (status 20))
 (segment (start 174.207401 115.458201) (end 174.1312 115.382) (width 0.1524) (layer F.Cu) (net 8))
 (segment (start 174.207401 117.107083) (end 174.207401 115.458201) (width 0.1524) (layer F.Cu) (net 8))
 (segment (start 174.935919 117.835601) (end 174.207401 117.107083) (width 0.1524) (layer F.Cu) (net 8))
 (segment (start 177.239799 117.835601) (end 174.935919 117.835601) (width 0.1524) (layer F.Cu) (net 8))
 (segment (start 177.7656 116.5098) (end 177.7656 117.3098) (width 0.1524) (layer F.Cu) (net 8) (status 10))
 (segment (start 177.7656 117.3098) (end 177.239799 117.835601) (width 0.1524) (layer F.Cu) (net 8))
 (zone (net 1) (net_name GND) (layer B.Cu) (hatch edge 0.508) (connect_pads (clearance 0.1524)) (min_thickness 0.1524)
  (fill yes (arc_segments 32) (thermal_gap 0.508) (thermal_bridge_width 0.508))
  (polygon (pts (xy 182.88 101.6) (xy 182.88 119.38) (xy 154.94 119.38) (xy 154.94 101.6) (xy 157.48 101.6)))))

